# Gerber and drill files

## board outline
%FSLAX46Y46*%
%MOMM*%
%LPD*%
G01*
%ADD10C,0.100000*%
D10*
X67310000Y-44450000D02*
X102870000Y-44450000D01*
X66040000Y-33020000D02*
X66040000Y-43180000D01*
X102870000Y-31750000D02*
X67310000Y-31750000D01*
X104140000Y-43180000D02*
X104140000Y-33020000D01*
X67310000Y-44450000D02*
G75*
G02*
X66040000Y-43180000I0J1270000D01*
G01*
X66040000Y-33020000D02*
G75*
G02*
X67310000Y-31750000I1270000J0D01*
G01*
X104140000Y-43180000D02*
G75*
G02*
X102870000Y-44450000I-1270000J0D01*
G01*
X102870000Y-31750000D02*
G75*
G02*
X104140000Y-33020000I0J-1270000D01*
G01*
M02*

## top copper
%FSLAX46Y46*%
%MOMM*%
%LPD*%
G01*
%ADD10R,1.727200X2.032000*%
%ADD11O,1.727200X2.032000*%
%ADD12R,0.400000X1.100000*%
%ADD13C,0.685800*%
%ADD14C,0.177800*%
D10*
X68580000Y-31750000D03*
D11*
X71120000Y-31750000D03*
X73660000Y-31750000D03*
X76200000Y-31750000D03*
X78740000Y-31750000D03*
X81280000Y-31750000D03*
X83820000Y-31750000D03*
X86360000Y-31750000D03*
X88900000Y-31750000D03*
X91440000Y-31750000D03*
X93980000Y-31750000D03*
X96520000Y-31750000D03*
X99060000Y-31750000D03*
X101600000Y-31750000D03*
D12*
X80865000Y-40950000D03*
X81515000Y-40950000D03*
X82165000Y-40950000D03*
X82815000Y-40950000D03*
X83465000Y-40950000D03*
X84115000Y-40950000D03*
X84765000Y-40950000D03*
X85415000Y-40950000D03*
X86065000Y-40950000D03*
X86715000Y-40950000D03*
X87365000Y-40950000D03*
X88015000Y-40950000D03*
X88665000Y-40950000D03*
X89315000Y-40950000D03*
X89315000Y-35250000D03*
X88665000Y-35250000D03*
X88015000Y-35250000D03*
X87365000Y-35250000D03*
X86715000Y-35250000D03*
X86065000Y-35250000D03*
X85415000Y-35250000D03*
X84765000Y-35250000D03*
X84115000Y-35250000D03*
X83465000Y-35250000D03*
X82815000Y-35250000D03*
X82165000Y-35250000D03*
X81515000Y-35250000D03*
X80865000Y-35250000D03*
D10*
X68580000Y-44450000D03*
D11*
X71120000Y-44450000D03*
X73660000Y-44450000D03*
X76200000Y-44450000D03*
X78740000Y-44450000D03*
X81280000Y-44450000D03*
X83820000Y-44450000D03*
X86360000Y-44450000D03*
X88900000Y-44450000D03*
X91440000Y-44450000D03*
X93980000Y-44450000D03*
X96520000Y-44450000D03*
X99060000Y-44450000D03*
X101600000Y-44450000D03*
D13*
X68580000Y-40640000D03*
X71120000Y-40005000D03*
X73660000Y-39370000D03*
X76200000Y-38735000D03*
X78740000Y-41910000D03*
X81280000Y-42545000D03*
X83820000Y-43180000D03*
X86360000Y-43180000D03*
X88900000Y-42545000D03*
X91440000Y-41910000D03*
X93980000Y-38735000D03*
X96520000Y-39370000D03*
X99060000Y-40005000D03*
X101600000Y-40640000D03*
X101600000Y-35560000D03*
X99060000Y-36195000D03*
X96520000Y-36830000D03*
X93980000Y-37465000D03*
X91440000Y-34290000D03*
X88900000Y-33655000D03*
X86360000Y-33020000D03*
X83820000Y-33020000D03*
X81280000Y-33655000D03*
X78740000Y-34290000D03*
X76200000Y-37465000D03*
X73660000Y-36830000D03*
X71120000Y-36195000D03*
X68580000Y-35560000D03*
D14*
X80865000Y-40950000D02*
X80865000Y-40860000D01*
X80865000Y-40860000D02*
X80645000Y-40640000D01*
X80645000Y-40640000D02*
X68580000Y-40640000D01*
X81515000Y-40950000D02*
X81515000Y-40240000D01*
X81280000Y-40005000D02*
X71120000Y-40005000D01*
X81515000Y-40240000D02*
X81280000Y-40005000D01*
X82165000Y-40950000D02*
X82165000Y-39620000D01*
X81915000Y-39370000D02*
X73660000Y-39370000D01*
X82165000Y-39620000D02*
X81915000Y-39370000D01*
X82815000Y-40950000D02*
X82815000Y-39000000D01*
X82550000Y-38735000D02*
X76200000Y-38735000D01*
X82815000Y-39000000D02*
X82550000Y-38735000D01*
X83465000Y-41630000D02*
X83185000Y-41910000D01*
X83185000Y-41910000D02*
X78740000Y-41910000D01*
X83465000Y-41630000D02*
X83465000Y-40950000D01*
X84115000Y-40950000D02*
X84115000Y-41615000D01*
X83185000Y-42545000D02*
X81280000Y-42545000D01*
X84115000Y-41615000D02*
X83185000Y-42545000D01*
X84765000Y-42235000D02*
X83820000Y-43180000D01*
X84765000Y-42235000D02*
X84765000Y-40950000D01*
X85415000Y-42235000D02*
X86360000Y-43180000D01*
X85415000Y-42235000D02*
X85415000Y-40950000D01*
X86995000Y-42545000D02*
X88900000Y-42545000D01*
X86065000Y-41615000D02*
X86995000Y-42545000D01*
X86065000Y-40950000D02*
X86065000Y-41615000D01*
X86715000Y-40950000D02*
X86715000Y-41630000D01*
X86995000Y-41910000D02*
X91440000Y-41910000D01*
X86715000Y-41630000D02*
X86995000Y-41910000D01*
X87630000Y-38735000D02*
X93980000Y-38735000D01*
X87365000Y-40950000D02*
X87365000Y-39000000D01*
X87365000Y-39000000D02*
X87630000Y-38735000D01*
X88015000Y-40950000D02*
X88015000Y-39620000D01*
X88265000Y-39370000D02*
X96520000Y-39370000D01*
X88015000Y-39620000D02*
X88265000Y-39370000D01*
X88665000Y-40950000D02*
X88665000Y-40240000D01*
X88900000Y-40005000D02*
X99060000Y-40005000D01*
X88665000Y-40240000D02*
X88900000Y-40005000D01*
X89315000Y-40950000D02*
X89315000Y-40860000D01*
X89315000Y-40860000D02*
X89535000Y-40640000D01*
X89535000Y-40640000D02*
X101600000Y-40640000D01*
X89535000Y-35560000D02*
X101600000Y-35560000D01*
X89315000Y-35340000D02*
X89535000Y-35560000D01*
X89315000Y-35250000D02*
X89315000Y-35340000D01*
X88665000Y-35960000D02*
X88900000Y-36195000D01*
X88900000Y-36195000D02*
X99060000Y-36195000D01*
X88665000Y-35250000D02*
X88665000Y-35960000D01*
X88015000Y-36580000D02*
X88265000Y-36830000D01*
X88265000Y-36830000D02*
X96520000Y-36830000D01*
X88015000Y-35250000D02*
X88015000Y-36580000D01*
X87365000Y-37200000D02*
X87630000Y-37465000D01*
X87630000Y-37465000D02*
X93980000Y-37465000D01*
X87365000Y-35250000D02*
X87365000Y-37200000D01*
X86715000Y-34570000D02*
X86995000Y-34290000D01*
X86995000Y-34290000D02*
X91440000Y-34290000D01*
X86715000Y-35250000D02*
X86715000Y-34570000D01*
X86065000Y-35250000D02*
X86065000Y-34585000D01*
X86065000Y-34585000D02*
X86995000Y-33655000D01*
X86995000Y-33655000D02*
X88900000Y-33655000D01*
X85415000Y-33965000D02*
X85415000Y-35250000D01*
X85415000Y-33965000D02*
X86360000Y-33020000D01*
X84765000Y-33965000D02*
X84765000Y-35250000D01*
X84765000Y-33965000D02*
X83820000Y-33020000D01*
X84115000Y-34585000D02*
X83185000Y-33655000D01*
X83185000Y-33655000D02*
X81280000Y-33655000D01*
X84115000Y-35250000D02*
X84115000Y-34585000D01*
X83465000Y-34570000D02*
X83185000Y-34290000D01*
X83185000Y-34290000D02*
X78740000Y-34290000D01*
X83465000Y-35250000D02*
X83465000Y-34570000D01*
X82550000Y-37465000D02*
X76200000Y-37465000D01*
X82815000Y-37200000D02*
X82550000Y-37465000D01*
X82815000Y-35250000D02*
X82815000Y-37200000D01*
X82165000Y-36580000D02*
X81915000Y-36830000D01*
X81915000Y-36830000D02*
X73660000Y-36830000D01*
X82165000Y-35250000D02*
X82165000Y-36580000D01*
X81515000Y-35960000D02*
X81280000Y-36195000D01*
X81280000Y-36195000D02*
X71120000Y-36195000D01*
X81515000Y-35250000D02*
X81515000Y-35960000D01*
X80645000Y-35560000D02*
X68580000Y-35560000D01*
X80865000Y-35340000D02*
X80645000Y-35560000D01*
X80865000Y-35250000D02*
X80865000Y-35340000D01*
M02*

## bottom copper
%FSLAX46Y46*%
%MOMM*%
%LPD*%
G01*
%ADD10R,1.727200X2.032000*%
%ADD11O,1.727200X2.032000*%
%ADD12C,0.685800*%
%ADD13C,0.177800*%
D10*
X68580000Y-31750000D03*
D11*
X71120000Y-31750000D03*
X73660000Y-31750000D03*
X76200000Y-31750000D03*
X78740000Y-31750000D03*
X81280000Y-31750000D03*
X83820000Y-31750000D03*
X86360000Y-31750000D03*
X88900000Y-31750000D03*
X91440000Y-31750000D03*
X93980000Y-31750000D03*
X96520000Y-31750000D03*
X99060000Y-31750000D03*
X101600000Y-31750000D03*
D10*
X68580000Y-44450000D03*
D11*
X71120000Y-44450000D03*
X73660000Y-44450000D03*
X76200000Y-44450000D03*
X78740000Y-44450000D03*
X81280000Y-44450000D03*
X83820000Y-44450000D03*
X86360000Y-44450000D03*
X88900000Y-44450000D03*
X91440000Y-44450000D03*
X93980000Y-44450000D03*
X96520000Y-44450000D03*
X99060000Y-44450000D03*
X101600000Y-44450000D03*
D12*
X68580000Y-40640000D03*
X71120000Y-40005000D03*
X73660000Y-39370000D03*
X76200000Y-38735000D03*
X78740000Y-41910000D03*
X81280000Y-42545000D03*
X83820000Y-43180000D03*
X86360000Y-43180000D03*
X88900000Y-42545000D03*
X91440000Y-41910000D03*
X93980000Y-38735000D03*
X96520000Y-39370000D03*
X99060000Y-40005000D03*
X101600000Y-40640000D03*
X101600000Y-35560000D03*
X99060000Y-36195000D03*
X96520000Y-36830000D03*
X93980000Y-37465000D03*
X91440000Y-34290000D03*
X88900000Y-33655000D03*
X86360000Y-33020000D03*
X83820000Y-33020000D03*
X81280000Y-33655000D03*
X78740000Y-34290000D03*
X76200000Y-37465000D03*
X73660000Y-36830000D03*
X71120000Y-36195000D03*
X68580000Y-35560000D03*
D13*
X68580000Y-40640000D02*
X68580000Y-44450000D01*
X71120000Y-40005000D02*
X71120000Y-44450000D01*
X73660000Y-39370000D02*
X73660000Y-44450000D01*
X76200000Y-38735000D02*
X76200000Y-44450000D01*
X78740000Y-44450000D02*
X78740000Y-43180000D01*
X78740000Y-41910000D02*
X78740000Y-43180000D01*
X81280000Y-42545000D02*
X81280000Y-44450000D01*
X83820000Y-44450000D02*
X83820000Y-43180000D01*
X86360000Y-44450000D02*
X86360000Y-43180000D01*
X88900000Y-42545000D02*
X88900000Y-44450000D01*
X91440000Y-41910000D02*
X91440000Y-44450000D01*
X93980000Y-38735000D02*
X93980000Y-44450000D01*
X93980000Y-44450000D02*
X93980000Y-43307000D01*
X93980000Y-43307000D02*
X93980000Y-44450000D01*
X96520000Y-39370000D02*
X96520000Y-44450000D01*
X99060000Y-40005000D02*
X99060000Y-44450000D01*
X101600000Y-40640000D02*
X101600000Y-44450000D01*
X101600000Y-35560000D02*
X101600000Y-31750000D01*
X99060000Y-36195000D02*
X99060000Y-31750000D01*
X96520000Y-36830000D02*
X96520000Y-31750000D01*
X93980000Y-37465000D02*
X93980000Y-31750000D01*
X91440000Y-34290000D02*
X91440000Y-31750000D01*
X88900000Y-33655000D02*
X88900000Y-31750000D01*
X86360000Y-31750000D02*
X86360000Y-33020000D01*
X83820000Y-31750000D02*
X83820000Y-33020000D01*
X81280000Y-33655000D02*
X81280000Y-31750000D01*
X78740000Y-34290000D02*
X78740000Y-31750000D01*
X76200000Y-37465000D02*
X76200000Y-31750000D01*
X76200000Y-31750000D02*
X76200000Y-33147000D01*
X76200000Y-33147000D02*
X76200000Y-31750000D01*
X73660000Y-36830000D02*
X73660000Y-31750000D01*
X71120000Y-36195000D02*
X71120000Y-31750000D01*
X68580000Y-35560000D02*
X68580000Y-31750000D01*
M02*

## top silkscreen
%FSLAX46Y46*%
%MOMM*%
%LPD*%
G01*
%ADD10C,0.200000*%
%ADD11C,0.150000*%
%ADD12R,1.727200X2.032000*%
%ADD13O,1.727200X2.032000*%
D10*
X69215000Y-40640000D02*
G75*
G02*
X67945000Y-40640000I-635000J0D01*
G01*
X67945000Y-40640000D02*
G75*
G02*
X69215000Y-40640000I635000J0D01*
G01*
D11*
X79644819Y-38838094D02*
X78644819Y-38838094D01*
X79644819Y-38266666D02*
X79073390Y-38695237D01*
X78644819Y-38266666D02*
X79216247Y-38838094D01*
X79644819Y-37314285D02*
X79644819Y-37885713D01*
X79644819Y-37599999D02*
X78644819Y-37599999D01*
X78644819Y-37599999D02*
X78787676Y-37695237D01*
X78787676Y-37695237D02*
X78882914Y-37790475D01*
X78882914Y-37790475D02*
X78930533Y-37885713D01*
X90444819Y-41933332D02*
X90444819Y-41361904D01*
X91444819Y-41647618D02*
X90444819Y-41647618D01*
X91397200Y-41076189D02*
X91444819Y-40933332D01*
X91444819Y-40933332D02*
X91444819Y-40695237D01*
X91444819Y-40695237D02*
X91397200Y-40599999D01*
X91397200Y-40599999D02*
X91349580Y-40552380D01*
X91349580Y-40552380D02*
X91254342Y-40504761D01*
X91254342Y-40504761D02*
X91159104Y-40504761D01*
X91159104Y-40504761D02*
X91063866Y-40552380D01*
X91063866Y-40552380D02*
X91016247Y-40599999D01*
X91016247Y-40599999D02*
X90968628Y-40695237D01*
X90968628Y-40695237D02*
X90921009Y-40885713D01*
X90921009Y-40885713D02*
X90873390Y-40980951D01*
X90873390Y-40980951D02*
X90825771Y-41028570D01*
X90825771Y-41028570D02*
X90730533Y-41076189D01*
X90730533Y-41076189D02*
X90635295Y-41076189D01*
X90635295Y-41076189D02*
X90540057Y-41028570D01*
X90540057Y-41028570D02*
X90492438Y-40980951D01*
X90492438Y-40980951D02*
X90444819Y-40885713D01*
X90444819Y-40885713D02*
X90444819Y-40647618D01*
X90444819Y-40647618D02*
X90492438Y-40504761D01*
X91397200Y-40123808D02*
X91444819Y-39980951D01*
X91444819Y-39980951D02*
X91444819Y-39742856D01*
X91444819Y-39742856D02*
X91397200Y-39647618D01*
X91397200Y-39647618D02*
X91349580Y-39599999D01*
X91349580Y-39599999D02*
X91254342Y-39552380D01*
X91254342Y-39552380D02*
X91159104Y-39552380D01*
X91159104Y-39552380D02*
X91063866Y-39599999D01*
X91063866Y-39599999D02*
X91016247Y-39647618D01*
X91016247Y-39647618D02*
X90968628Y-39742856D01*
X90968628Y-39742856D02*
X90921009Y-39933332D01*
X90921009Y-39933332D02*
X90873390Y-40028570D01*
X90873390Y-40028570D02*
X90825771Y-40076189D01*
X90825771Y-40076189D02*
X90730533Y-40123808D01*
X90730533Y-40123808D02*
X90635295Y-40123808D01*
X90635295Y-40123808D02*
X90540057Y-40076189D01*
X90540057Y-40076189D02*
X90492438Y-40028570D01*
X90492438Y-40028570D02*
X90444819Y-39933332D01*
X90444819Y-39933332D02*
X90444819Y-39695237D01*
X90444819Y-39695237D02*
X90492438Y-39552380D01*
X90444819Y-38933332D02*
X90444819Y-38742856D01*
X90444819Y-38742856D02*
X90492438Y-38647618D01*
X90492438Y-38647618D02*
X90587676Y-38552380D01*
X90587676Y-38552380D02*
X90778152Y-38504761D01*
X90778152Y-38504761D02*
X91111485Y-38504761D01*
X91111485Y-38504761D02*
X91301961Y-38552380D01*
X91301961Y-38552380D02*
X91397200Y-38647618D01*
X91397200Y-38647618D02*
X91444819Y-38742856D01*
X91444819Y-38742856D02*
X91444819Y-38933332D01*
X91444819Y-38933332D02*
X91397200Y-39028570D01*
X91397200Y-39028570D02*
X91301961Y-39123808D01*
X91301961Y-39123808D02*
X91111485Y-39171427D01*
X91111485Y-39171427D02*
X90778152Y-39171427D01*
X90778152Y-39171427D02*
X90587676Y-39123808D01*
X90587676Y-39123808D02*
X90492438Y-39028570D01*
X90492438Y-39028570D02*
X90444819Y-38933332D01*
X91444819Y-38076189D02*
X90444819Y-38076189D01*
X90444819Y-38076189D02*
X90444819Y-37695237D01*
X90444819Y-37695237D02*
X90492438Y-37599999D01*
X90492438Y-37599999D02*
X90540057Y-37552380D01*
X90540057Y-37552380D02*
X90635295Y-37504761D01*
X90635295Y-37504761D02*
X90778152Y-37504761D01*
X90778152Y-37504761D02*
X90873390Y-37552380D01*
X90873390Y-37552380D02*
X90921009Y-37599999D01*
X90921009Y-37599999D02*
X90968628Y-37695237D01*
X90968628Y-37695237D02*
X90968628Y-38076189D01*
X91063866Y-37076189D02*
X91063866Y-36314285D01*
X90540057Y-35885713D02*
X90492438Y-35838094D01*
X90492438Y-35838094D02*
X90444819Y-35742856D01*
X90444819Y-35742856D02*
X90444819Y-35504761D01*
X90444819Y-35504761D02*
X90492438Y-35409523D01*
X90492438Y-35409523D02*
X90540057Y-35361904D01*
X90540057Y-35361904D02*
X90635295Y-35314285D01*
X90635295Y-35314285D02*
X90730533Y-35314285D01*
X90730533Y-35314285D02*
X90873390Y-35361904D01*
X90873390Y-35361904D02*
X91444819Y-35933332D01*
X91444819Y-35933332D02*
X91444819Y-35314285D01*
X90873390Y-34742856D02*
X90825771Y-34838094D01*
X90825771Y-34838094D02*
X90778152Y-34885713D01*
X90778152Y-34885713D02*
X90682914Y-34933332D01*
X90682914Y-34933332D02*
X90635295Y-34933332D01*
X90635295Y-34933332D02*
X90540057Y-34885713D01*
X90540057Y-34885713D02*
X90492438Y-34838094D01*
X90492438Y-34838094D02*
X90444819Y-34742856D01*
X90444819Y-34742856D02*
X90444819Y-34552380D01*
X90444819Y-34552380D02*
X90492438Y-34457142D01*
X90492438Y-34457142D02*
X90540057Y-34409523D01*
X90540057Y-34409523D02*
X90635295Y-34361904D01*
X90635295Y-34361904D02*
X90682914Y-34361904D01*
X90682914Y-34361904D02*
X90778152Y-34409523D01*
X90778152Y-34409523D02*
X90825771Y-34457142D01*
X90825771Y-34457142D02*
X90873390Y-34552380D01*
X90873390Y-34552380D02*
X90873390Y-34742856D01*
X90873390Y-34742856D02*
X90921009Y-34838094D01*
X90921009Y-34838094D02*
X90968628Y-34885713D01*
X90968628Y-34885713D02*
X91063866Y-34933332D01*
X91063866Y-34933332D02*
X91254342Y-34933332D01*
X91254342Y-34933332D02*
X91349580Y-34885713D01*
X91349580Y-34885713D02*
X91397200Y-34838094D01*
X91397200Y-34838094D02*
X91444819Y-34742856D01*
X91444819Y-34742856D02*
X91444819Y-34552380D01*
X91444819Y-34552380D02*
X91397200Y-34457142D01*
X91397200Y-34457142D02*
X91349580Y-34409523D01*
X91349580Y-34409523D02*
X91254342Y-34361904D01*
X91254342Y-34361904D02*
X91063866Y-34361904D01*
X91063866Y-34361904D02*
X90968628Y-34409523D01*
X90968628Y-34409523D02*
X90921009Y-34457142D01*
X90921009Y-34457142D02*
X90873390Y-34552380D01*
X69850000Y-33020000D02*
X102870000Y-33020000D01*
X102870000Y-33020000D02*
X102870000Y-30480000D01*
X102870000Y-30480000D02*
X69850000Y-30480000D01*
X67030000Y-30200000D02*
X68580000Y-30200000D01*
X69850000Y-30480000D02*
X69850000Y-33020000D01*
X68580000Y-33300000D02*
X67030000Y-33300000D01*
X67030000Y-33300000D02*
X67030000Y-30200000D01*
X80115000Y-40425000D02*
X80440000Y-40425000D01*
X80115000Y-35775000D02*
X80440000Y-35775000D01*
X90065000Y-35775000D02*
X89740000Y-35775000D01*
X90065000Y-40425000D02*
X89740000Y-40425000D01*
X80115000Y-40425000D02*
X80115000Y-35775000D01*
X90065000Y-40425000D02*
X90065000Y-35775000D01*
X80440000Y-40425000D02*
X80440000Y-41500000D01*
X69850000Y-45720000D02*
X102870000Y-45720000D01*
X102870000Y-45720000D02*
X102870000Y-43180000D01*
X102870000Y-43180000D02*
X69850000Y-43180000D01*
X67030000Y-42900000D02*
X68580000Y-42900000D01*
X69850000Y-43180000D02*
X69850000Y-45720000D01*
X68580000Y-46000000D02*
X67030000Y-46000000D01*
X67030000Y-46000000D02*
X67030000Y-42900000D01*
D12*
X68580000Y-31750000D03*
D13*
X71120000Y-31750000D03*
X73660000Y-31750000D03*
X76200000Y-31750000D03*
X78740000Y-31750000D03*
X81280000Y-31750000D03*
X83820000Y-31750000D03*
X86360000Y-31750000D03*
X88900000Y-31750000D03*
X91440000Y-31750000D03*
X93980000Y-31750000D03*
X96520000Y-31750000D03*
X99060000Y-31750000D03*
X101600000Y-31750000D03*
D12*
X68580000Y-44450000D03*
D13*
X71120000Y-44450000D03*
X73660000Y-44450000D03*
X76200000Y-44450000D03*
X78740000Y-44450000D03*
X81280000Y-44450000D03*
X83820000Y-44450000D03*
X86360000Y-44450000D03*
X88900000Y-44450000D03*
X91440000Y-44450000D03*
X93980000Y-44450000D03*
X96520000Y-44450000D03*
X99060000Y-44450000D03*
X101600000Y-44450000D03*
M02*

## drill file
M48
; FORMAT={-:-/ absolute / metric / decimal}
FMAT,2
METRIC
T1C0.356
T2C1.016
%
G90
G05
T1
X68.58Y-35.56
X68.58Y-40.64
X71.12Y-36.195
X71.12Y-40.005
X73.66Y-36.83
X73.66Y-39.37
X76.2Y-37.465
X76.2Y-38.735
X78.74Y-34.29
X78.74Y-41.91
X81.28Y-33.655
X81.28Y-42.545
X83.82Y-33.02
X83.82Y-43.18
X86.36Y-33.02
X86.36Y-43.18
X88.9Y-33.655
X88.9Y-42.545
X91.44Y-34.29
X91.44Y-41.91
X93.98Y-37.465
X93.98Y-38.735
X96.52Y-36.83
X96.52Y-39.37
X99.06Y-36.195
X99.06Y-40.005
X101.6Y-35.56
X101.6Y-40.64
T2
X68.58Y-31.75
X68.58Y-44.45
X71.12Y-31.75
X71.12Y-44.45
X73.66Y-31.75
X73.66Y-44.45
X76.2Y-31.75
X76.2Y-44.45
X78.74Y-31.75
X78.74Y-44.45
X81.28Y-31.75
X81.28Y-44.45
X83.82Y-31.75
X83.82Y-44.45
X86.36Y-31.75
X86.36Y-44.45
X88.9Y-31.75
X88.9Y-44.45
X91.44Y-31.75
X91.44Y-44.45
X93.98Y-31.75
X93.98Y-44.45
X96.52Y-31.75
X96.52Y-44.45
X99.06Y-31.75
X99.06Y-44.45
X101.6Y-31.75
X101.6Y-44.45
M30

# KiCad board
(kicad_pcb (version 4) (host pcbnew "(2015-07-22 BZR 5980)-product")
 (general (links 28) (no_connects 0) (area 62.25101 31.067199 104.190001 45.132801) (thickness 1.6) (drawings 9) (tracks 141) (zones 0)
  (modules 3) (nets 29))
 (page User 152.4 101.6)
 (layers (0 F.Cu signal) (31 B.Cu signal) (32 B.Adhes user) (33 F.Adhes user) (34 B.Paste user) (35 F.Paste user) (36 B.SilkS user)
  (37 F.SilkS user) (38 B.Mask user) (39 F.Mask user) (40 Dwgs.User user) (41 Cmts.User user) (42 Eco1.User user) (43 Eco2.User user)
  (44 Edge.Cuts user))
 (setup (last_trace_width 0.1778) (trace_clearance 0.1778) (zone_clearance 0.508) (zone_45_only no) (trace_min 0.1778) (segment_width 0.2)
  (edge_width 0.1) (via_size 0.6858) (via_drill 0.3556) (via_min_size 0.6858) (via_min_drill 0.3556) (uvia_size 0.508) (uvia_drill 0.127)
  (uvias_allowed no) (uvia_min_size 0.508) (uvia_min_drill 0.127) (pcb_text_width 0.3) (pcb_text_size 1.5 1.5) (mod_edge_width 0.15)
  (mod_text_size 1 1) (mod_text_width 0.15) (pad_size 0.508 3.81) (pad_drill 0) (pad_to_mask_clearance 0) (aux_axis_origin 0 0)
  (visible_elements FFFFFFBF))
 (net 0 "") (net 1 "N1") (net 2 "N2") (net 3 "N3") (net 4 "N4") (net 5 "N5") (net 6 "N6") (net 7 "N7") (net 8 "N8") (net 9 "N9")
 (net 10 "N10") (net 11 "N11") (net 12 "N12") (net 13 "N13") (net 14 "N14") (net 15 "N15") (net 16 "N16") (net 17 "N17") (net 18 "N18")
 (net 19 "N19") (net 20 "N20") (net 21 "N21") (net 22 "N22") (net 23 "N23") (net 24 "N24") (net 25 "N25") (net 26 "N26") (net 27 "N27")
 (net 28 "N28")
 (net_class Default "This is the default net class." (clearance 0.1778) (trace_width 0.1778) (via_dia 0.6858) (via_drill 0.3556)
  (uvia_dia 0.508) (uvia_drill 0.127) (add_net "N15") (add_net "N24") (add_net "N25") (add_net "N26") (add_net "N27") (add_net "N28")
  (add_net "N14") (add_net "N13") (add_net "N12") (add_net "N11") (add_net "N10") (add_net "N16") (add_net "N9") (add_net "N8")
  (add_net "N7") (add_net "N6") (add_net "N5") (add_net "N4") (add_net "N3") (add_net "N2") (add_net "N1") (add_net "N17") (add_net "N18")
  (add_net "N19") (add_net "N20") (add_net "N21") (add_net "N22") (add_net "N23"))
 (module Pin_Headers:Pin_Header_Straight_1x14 (layer F.Cu) (at 68.58 31.75 90)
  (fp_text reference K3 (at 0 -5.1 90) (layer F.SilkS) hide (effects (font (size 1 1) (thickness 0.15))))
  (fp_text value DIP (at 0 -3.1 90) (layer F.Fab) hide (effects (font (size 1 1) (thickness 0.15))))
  (fp_line (start -1.27 1.27) (end -1.27 34.29) (layer F.SilkS) (width 0.15))
  (fp_line (start -1.27 34.29) (end 1.27 34.29) (layer F.SilkS) (width 0.15))
  (fp_line (start 1.27 34.29) (end 1.27 1.27) (layer F.SilkS) (width 0.15))
  (fp_line (start 1.55 -1.55) (end 1.55 0) (layer F.SilkS) (width 0.15))
  (fp_line (start 1.27 1.27) (end -1.27 1.27) (layer F.SilkS) (width 0.15))
  (fp_line (start -1.55 0) (end -1.55 -1.55) (layer F.SilkS) (width 0.15))
  (fp_line (start -1.55 -1.55) (end 1.55 -1.55) (layer F.SilkS) (width 0.15))
  (pad 1 thru_hole rect (at 0 0 90) (size 2.032 1.7272) (drill 1.016) (layers *.Cu *.Mask F.SilkS) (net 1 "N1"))
  (pad 2 thru_hole oval (at 0 2.54 90) (size 2.032 1.7272) (drill 1.016) (layers *.Cu *.Mask F.SilkS) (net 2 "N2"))
  (pad 3 thru_hole oval (at 0 5.08 90) (size 2.032 1.7272) (drill 1.016) (layers *.Cu *.Mask F.SilkS) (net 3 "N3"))
  (pad 4 thru_hole oval (at 0 7.62 90) (size 2.032 1.7272) (drill 1.016) (layers *.Cu *.Mask F.SilkS) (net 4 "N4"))
  (pad 5 thru_hole oval (at 0 10.16 90) (size 2.032 1.7272) (drill 1.016) (layers *.Cu *.Mask F.SilkS) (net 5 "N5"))
  (pad 6 thru_hole oval (at 0 12.7 90) (size 2.032 1.7272) (drill 1.016) (layers *.Cu *.Mask F.SilkS) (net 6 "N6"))
  (pad 7 thru_hole oval (at 0 15.24 90) (size 2.032 1.7272) (drill 1.016) (layers *.Cu *.Mask F.SilkS) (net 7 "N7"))
  (pad 8 thru_hole oval (at 0 17.78 90) (size 2.032 1.7272) (drill 1.016) (layers *.Cu *.Mask F.SilkS) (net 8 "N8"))
  (pad 9 thru_hole oval (at 0 20.32 90) (size 2.032 1.7272) (drill 1.016) (layers *.Cu *.Mask F.SilkS) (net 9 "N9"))
  (pad 10 thru_hole oval (at 0 22.86 90) (size 2.032 1.7272) (drill 1.016) (layers *.Cu *.Mask F.SilkS) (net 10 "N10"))
  (pad 11 thru_hole oval (at 0 25.4 90) (size 2.032 1.7272) (drill 1.016) (layers *.Cu *.Mask F.SilkS) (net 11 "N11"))
  (pad 12 thru_hole oval (at 0 27.94 90) (size 2.032 1.7272) (drill 1.016) (layers *.Cu *.Mask F.SilkS) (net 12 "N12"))
  (pad 13 thru_hole oval (at 0 30.48 90) (size 2.032 1.7272) (drill 1.016) (layers *.Cu *.Mask F.SilkS) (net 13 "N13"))
  (pad 14 thru_hole oval (at 0 33.02 90) (size 2.032 1.7272) (drill 1.016) (layers *.Cu *.Mask F.SilkS) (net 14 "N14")))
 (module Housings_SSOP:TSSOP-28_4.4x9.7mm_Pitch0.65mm (layer F.Cu) (at 85.09 38.1 90)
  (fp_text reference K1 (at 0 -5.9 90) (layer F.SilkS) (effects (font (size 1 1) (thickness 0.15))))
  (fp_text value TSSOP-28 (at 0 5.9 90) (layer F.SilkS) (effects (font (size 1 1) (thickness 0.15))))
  (fp_line (start -2.325 -4.975) (end -2.325 -4.65) (layer F.SilkS) (width 0.15))
  (fp_line (start 2.325 -4.975) (end 2.325 -4.65) (layer F.SilkS) (width 0.15))
  (fp_line (start 2.325 4.975) (end 2.325 4.65) (layer F.SilkS) (width 0.15))
  (fp_line (start -2.325 4.975) (end -2.325 4.65) (layer F.SilkS) (width 0.15))
  (fp_line (start -2.325 -4.975) (end 2.325 -4.975) (layer F.SilkS) (width 0.15))
  (fp_line (start -2.325 4.975) (end 2.325 4.975) (layer F.SilkS) (width 0.15))
  (fp_line (start -2.325 -4.65) (end -3.4 -4.65) (layer F.SilkS) (width 0.15))
  (pad 1 smd rect (at -2.85 -4.225 90) (size 1.1 0.4) (layers F.Cu F.Paste F.Mask) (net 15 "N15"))
  (pad 2 smd rect (at -2.85 -3.575 90) (size 1.1 0.4) (layers F.Cu F.Paste F.Mask) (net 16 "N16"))
  (pad 3 smd rect (at -2.85 -2.925 90) (size 1.1 0.4) (layers F.Cu F.Paste F.Mask) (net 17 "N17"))
  (pad 4 smd rect (at -2.85 -2.275 90) (size 1.1 0.4) (layers F.Cu F.Paste F.Mask) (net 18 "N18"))
  (pad 5 smd rect (at -2.85 -1.625 90) (size 1.1 0.4) (layers F.Cu F.Paste F.Mask) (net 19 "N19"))
  (pad 6 smd rect (at -2.85 -0.975 90) (size 1.1 0.4) (layers F.Cu F.Paste F.Mask) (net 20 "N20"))
  (pad 7 smd rect (at -2.85 -0.325 90) (size 1.1 0.4) (layers F.Cu F.Paste F.Mask) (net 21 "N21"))
  (pad 8 smd rect (at -2.85 0.325 90) (size 1.1 0.4) (layers F.Cu F.Paste F.Mask) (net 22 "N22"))
  (pad 9 smd rect (at -2.85 0.975 90) (size 1.1 0.4) (layers F.Cu F.Paste F.Mask) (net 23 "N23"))
  (pad 10 smd rect (at -2.85 1.625 90) (size 1.1 0.4) (layers F.Cu F.Paste F.Mask) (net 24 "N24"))
  (pad 11 smd rect (at -2.85 2.275 90) (size 1.1 0.4) (layers F.Cu F.Paste F.Mask) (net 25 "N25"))
  (pad 12 smd rect (at -2.85 2.925 90) (size 1.1 0.4) (layers F.Cu F.Paste F.Mask) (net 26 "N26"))
  (pad 13 smd rect (at -2.85 3.575 90) (size 1.1 0.4) (layers F.Cu F.Paste F.Mask) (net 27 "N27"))
  (pad 14 smd rect (at -2.85 4.225 90) (size 1.1 0.4) (layers F.Cu F.Paste F.Mask) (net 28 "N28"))
  (pad 15 smd rect (at 2.85 4.225 90) (size 1.1 0.4) (layers F.Cu F.Paste F.Mask) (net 14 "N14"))
  (pad 16 smd rect (at 2.85 3.575 90) (size 1.1 0.4) (layers F.Cu F.Paste F.Mask) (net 13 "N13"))
  (pad 17 smd rect (at 2.85 2.925 90) (size 1.1 0.4) (layers F.Cu F.Paste F.Mask) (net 12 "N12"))
  (pad 18 smd rect (at 2.85 2.275 90) (size 1.1 0.4) (layers F.Cu F.Paste F.Mask) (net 11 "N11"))
  (pad 19 smd rect (at 2.85 1.625 90) (size 1.1 0.4) (layers F.Cu F.Paste F.Mask) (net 10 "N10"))
  (pad 20 smd rect (at 2.85 0.975 90) (size 1.1 0.4) (layers F.Cu F.Paste F.Mask) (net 9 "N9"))
  (pad 21 smd rect (at 2.85 0.325 90) (size 1.1 0.4) (layers F.Cu F.Paste F.Mask) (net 8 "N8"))
  (pad 22 smd rect (at 2.85 -0.325 90) (size 1.1 0.4) (layers F.Cu F.Paste F.Mask) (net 7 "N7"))
  (pad 23 smd rect (at 2.85 -0.975 90) (size 1.1 0.4) (layers F.Cu F.Paste F.Mask) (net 6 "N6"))
  (pad 24 smd rect (at 2.85 -1.625 90) (size 1.1 0.4) (layers F.Cu F.Paste F.Mask) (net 5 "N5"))
  (pad 25 smd rect (at 2.85 -2.275 90) (size 1.1 0.4) (layers F.Cu F.Paste F.Mask) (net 4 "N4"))
  (pad 26 smd rect (at 2.85 -2.925 90) (size 1.1 0.4) (layers F.Cu F.Paste F.Mask) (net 3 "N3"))
  (pad 27 smd rect (at 2.85 -3.575 90) (size 1.1 0.4) (layers F.Cu F.Paste F.Mask) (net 2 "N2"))
  (pad 28 smd rect (at 2.85 -4.225 90) (size 1.1 0.4) (layers F.Cu F.Paste F.Mask) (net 1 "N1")))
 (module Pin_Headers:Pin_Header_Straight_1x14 (layer F.Cu) (at 68.58 44.45 90)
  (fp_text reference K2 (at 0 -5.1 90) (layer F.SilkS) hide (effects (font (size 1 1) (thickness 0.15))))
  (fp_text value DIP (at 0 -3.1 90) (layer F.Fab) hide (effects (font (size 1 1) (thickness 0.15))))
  (fp_line (start -1.27 1.27) (end -1.27 34.29) (layer F.SilkS) (width 0.15))
  (fp_line (start -1.27 34.29) (end 1.27 34.29) (layer F.SilkS) (width 0.15))
  (fp_line (start 1.27 34.29) (end 1.27 1.27) (layer F.SilkS) (width 0.15))
  (fp_line (start 1.55 -1.55) (end 1.55 0) (layer F.SilkS) (width 0.15))
  (fp_line (start 1.27 1.27) (end -1.27 1.27) (layer F.SilkS) (width 0.15))
  (fp_line (start -1.55 0) (end -1.55 -1.55) (layer F.SilkS) (width 0.15))
  (fp_line (start -1.55 -1.55) (end 1.55 -1.55) (layer F.SilkS) (width 0.15))
  (pad 1 thru_hole rect (at 0 0 90) (size 2.032 1.7272) (drill 1.016) (layers *.Cu *.Mask F.SilkS) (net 15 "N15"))
  (pad 2 thru_hole oval (at 0 2.54 90) (size 2.032 1.7272) (drill 1.016) (layers *.Cu *.Mask F.SilkS) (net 16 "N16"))
  (pad 3 thru_hole oval (at 0 5.08 90) (size 2.032 1.7272) (drill 1.016) (layers *.Cu *.Mask F.SilkS) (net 17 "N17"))
  (pad 4 thru_hole oval (at 0 7.62 90) (size 2.032 1.7272) (drill 1.016) (layers *.Cu *.Mask F.SilkS) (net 18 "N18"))
  (pad 5 thru_hole oval (at 0 10.16 90) (size 2.032 1.7272) (drill 1.016) (layers *.Cu *.Mask F.SilkS) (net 19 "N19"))
  (pad 6 thru_hole oval (at 0 12.7 90) (size 2.032 1.7272) (drill 1.016) (layers *.Cu *.Mask F.SilkS) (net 20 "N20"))
  (pad 7 thru_hole oval (at 0 15.24 90) (size 2.032 1.7272) (drill 1.016) (layers *.Cu *.Mask F.SilkS) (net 21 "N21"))
  (pad 8 thru_hole oval (at 0 17.78 90) (size 2.032 1.7272) (drill 1.016) (layers *.Cu *.Mask F.SilkS) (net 22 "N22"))
  (pad 9 thru_hole oval (at 0 20.32 90) (size 2.032 1.7272) (drill 1.016) (layers *.Cu *.Mask F.SilkS) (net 23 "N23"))
  (pad 10 thru_hole oval (at 0 22.86 90) (size 2.032 1.7272) (drill 1.016) (layers *.Cu *.Mask F.SilkS) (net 24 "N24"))
  (pad 11 thru_hole oval (at 0 25.4 90) (size 2.032 1.7272) (drill 1.016) (layers *.Cu *.Mask F.SilkS) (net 25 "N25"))
  (pad 12 thru_hole oval (at 0 27.94 90) (size 2.032 1.7272) (drill 1.016) (layers *.Cu *.Mask F.SilkS) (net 26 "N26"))
  (pad 13 thru_hole oval (at 0 30.48 90) (size 2.032 1.7272) (drill 1.016) (layers *.Cu *.Mask F.SilkS) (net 27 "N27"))
  (pad 14 thru_hole oval (at 0 33.02 90) (size 2.032 1.7272) (drill 1.016) (layers *.Cu *.Mask F.SilkS) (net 28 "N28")))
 (gr_circle (center 68.58 40.64) (end 68.58 40.005) (layer F.SilkS) (width 0.2))
 (gr_line (start 67.31 44.45) (end 102.87 44.45) (angle 90) (layer Edge.Cuts) (width 0.1))
 (gr_line (start 66.04 33.02) (end 66.04 43.18) (angle 90) (layer Edge.Cuts) (width 0.1))
 (gr_line (start 102.87 31.75) (end 67.31 31.75) (angle 90) (layer Edge.Cuts) (width 0.1))
 (gr_line (start 104.14 43.18) (end 104.14 33.02) (angle 90) (layer Edge.Cuts) (width 0.1))
 (gr_arc (start 67.31 43.18) (end 67.31 44.45) (angle 90) (layer Edge.Cuts) (width 0.1))
 (gr_arc (start 67.31 33.02) (end 66.04 33.02) (angle 90) (layer Edge.Cuts) (width 0.1))
 (gr_arc (start 102.87 43.18) (end 104.14 43.18) (angle 90) (layer Edge.Cuts) (width 0.1))
 (gr_arc (start 102.87 33.02) (end 102.87 31.75) (angle 90) (layer Edge.Cuts) (width 0.1))
 (segment (start 80.865 40.95) (end 80.865 40.86) (width 0.1778) (layer F.Cu) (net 15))
 (segment (start 80.865 40.86) (end 80.645 40.64) (width 0.1778) (layer F.Cu) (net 15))
 (segment (start 68.58 40.64) (end 68.58 44.45) (width 0.1778) (layer B.Cu) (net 15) (status 800000))
 (via (at 68.58 40.64) (size 0.6858) (drill 0.3556) (layers F.Cu B.Cu) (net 15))
 (segment (start 80.645 40.64) (end 68.58 40.64) (width 0.1778) (layer F.Cu) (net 15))
 (segment (start 81.515 40.95) (end 81.515 40.24) (width 0.1778) (layer F.Cu) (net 16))
 (segment (start 71.12 40.005) (end 71.12 44.45) (width 0.1778) (layer B.Cu) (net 16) (status 800000))
 (via (at 71.12 40.005) (size 0.6858) (drill 0.3556) (layers F.Cu B.Cu) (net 16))
 (segment (start 81.28 40.005) (end 71.12 40.005) (width 0.1778) (layer F.Cu) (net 16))
 (segment (start 81.515 40.24) (end 81.28 40.005) (width 0.1778) (layer F.Cu) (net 16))
 (segment (start 82.165 40.95) (end 82.165 39.62) (width 0.1778) (layer F.Cu) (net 17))
 (segment (start 73.66 39.37) (end 73.66 44.45) (width 0.1778) (layer B.Cu) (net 17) (status 800000))
 (via (at 73.66 39.37) (size 0.6858) (drill 0.3556) (layers F.Cu B.Cu) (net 17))
 (segment (start 81.915 39.37) (end 73.66 39.37) (width 0.1778) (layer F.Cu) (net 17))
 (segment (start 82.165 39.62) (end 81.915 39.37) (width 0.1778) (layer F.Cu) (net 17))
 (segment (start 82.815 40.95) (end 82.815 39) (width 0.1778) (layer F.Cu) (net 18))
 (segment (start 76.2 38.735) (end 76.2 44.45) (width 0.1778) (layer B.Cu) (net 18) (status 800000))
 (via (at 76.2 38.735) (size 0.6858) (drill 0.3556) (layers F.Cu B.Cu) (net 18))
 (segment (start 82.55 38.735) (end 76.2 38.735) (width 0.1778) (layer F.Cu) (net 18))
 (segment (start 82.815 39) (end 82.55 38.735) (width 0.1778) (layer F.Cu) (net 18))
 (segment (start 78.74 44.45) (end 78.74 43.18) (width 0.1778) (layer B.Cu) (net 19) (status 400000))
 (segment (start 83.465 41.63) (end 83.185 41.91) (width 0.1778) (layer F.Cu) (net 19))
 (segment (start 83.185 41.91) (end 78.74 41.91) (width 0.1778) (layer F.Cu) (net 19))
 (via (at 78.74 41.91) (size 0.6858) (drill 0.3556) (layers F.Cu B.Cu) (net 19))
 (segment (start 78.74 41.91) (end 78.74 43.18) (width 0.1778) (layer B.Cu) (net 19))
 (segment (start 83.465 41.63) (end 83.465 40.95) (width 0.1778) (layer F.Cu) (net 19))
 (segment (start 84.115 40.95) (end 84.115 41.615) (width 0.1778) (layer F.Cu) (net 20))
 (segment (start 81.28 42.545) (end 81.28 44.45) (width 0.1778) (layer B.Cu) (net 20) (status 800000))
 (via (at 81.28 42.545) (size 0.6858) (drill 0.3556) (layers F.Cu B.Cu) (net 20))
 (segment (start 83.185 42.545) (end 81.28 42.545) (width 0.1778) (layer F.Cu) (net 20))
 (segment (start 84.115 41.615) (end 83.185 42.545) (width 0.1778) (layer F.Cu) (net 20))
 (segment (start 83.82 44.45) (end 83.82 43.18) (width 0.1778) (layer B.Cu) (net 21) (status 400000))
 (segment (start 84.765 42.235) (end 83.82 43.18) (width 0.1778) (layer F.Cu) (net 21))
 (via (at 83.82 43.18) (size 0.6858) (drill 0.3556) (layers F.Cu B.Cu) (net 21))
 (segment (start 84.765 42.235) (end 84.765 40.95) (width 0.1778) (layer F.Cu) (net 21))
 (segment (start 86.36 44.45) (end 86.36 43.18) (width 0.1778) (layer B.Cu) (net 22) (status 400000))
 (segment (start 85.415 42.235) (end 86.36 43.18) (width 0.1778) (layer F.Cu) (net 22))
 (via (at 86.36 43.18) (size 0.6858) (drill 0.3556) (layers F.Cu B.Cu) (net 22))
 (segment (start 85.415 42.235) (end 85.415 40.95) (width 0.1778) (layer F.Cu) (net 22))
 (segment (start 86.995 42.545) (end 88.9 42.545) (width 0.1778) (layer F.Cu) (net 23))
 (segment (start 86.065 41.615) (end 86.995 42.545) (width 0.1778) (layer F.Cu) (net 23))
 (segment (start 86.065 40.95) (end 86.065 41.615) (width 0.1778) (layer F.Cu) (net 23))
 (segment (start 88.9 42.545) (end 88.9 44.45) (width 0.1778) (layer B.Cu) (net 23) (status 800000))
 (via (at 88.9 42.545) (size 0.6858) (drill 0.3556) (layers F.Cu B.Cu) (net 23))
 (segment (start 86.715 40.95) (end 86.715 41.63) (width 0.1778) (layer F.Cu) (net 24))
 (segment (start 91.44 41.91) (end 91.44 44.45) (width 0.1778) (layer B.Cu) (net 24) (status 800000))
 (via (at 91.44 41.91) (size 0.6858) (drill 0.3556) (layers F.Cu B.Cu) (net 24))
 (segment (start 86.995 41.91) (end 91.44 41.91) (width 0.1778) (layer F.Cu) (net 24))
 (segment (start 86.715 41.63) (end 86.995 41.91) (width 0.1778) (layer F.Cu) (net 24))
 (segment (start 87.63 38.735) (end 93.98 38.735) (width 0.1778) (layer F.Cu) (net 25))
 (segment (start 93.98 38.735) (end 93.98 44.45) (width 0.1778) (layer B.Cu) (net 25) (status 800000))
 (via (at 93.98 38.735) (size 0.6858) (drill 0.3556) (layers F.Cu B.Cu) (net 25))
 (segment (start 93.98 44.45) (end 93.98 43.307) (width 0.1778) (layer B.Cu) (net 25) (status 400000))
 (segment (start 93.98 43.307) (end 93.98 44.45) (width 0.1778) (layer B.Cu) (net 25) (status 800000))
 (segment (start 87.365 40.95) (end 87.365 39) (width 0.1778) (layer F.Cu) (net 25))
 (segment (start 87.365 39) (end 87.63 38.735) (width 0.1778) (layer F.Cu) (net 25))
 (segment (start 88.015 40.95) (end 88.015 39.62) (width 0.1778) (layer F.Cu) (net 26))
 (segment (start 96.52 39.37) (end 96.52 44.45) (width 0.1778) (layer B.Cu) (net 26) (status 800000))
 (via (at 96.52 39.37) (size 0.6858) (drill 0.3556) (layers F.Cu B.Cu) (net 26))
 (segment (start 88.265 39.37) (end 96.52 39.37) (width 0.1778) (layer F.Cu) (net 26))
 (segment (start 88.015 39.62) (end 88.265 39.37) (width 0.1778) (layer F.Cu) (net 26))
 (segment (start 88.665 40.95) (end 88.665 40.24) (width 0.1778) (layer F.Cu) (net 27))
 (segment (start 99.06 40.005) (end 99.06 44.45) (width 0.1778) (layer B.Cu) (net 27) (status 800000))
 (via (at 99.06 40.005) (size 0.6858) (drill 0.3556) (layers F.Cu B.Cu) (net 27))
 (segment (start 88.9 40.005) (end 99.06 40.005) (width 0.1778) (layer F.Cu) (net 27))
 (segment (start 88.665 40.24) (end 88.9 40.005) (width 0.1778) (layer F.Cu) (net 27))
 (segment (start 89.315 40.95) (end 89.315 40.86) (width 0.1778) (layer F.Cu) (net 28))
 (segment (start 89.315 40.86) (end 89.535 40.64) (width 0.1778) (layer F.Cu) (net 28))
 (segment (start 89.535 40.64) (end 101.6 40.64) (width 0.1778) (layer F.Cu) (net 28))
 (via (at 101.6 40.64) (size 0.6858) (drill 0.3556) (layers F.Cu B.Cu) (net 28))
 (segment (start 101.6 40.64) (end 101.6 44.45) (width 0.1778) (layer B.Cu) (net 28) (status 800000))
 (segment (start 89.535 35.56) (end 101.6 35.56) (width 0.1778) (layer F.Cu) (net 14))
 (via (at 101.6 35.56) (size 0.6858) (drill 0.3556) (layers F.Cu B.Cu) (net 14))
 (segment (start 101.6 35.56) (end 101.6 31.75) (width 0.1778) (layer B.Cu) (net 14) (status 800000))
 (segment (start 89.315 35.34) (end 89.535 35.56) (width 0.1778) (layer F.Cu) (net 14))
 (segment (start 89.315 35.25) (end 89.315 35.34) (width 0.1778) (layer F.Cu) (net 14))
 (segment (start 88.665 35.96) (end 88.9 36.195) (width 0.1778) (layer F.Cu) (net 13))
 (segment (start 88.9 36.195) (end 99.06 36.195) (width 0.1778) (layer F.Cu) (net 13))
 (via (at 99.06 36.195) (size 0.6858) (drill 0.3556) (layers F.Cu B.Cu) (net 13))
 (segment (start 99.06 36.195) (end 99.06 31.75) (width 0.1778) (layer B.Cu) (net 13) (status 800000))
 (segment (start 88.665 35.25) (end 88.665 35.96) (width 0.1778) (layer F.Cu) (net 13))
 (segment (start 88.015 36.58) (end 88.265 36.83) (width 0.1778) (layer F.Cu) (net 12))
 (segment (start 88.265 36.83) (end 96.52 36.83) (width 0.1778) (layer F.Cu) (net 12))
 (via (at 96.52 36.83) (size 0.6858) (drill 0.3556) (layers F.Cu B.Cu) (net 12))
 (segment (start 96.52 36.83) (end 96.52 31.75) (width 0.1778) (layer B.Cu) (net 12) (status 800000))
 (segment (start 88.015 35.25) (end 88.015 36.58) (width 0.1778) (layer F.Cu) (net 12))
 (segment (start 87.365 37.2) (end 87.63 37.465) (width 0.1778) (layer F.Cu) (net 11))
 (segment (start 87.63 37.465) (end 93.98 37.465) (width 0.1778) (layer F.Cu) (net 11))
 (via (at 93.98 37.465) (size 0.6858) (drill 0.3556) (layers F.Cu B.Cu) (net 11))
 (segment (start 93.98 37.465) (end 93.98 31.75) (width 0.1778) (layer B.Cu) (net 11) (status 800000))
 (segment (start 87.365 35.25) (end 87.365 37.2) (width 0.1778) (layer F.Cu) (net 11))
 (segment (start 86.715 34.57) (end 86.995 34.29) (width 0.1778) (layer F.Cu) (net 10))
 (segment (start 86.995 34.29) (end 91.44 34.29) (width 0.1778) (layer F.Cu) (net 10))
 (via (at 91.44 34.29) (size 0.6858) (drill 0.3556) (layers F.Cu B.Cu) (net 10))
 (segment (start 91.44 34.29) (end 91.44 31.75) (width 0.1778) (layer B.Cu) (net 10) (status 800000))
 (segment (start 86.715 35.25) (end 86.715 34.57) (width 0.1778) (layer F.Cu) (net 10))
 (via (at 88.9 33.655) (size 0.6858) (drill 0.3556) (layers F.Cu B.Cu) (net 9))
 (segment (start 88.9 33.655) (end 88.9 31.75) (width 0.1778) (layer B.Cu) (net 9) (status 800000))
 (segment (start 86.065 35.25) (end 86.065 34.585) (width 0.1778) (layer F.Cu) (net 9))
 (segment (start 86.065 34.585) (end 86.995 33.655) (width 0.1778) (layer F.Cu) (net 9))
 (segment (start 86.995 33.655) (end 88.9 33.655) (width 0.1778) (layer F.Cu) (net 9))
 (segment (start 86.36 31.75) (end 86.36 33.02) (width 0.1778) (layer B.Cu) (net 8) (status 400000))
 (segment (start 85.415 33.965) (end 85.415 35.25) (width 0.1778) (layer F.Cu) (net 8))
 (via (at 86.36 33.02) (size 0.6858) (drill 0.3556) (layers F.Cu B.Cu) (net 8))
 (segment (start 85.415 33.965) (end 86.36 33.02) (width 0.1778) (layer F.Cu) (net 8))
 (segment (start 83.82 31.75) (end 83.82 33.02) (width 0.1778) (layer B.Cu) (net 7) (status 400000))
 (segment (start 84.765 33.965) (end 84.765 35.25) (width 0.1778) (layer F.Cu) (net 7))
 (via (at 83.82 33.02) (size 0.6858) (drill 0.3556) (layers F.Cu B.Cu) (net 7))
 (segment (start 84.765 33.965) (end 83.82 33.02) (width 0.1778) (layer F.Cu) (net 7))
 (segment (start 84.115 34.585) (end 83.185 33.655) (width 0.1778) (layer F.Cu) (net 6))
 (segment (start 83.185 33.655) (end 81.28 33.655) (width 0.1778) (layer F.Cu) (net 6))
 (via (at 81.28 33.655) (size 0.6858) (drill 0.3556) (layers F.Cu B.Cu) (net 6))
 (segment (start 81.28 33.655) (end 81.28 31.75) (width 0.1778) (layer B.Cu) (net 6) (status 800000))
 (segment (start 84.115 35.25) (end 84.115 34.585) (width 0.1778) (layer F.Cu) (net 6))
 (segment (start 83.465 34.57) (end 83.185 34.29) (width 0.1778) (layer F.Cu) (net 5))
 (segment (start 83.185 34.29) (end 78.74 34.29) (width 0.1778) (layer F.Cu) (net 5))
 (via (at 78.74 34.29) (size 0.6858) (drill 0.3556) (layers F.Cu B.Cu) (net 5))
 (segment (start 78.74 34.29) (end 78.74 31.75) (width 0.1778) (layer B.Cu) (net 5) (status 800000))
 (segment (start 83.465 35.25) (end 83.465 34.57) (width 0.1778) (layer F.Cu) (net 5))
 (segment (start 82.55 37.465) (end 76.2 37.465) (width 0.1778) (layer F.Cu) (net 4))
 (segment (start 76.2 37.465) (end 76.2 31.75) (width 0.1778) (layer B.Cu) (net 4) (status 800000))
 (via (at 76.2 37.465) (size 0.6858) (drill 0.3556) (layers F.Cu B.Cu) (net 4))
 (segment (start 76.2 31.75) (end 76.2 33.147) (width 0.1778) (layer B.Cu) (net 4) (status 400000))
 (segment (start 76.2 33.147) (end 76.2 31.75) (width 0.1778) (layer B.Cu) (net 4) (status 800000))
 (segment (start 82.815 37.2) (end 82.55 37.465) (width 0.1778) (layer F.Cu) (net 4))
 (segment (start 82.815 35.25) (end 82.815 37.2) (width 0.1778) (layer F.Cu) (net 4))
 (segment (start 82.165 36.58) (end 81.915 36.83) (width 0.1778) (layer F.Cu) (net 3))
 (segment (start 81.915 36.83) (end 73.66 36.83) (width 0.1778) (layer F.Cu) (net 3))
 (via (at 73.66 36.83) (size 0.6858) (drill 0.3556) (layers F.Cu B.Cu) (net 3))
 (segment (start 73.66 36.83) (end 73.66 31.75) (width 0.1778) (layer B.Cu) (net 3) (status 800000))
 (segment (start 82.165 35.25) (end 82.165 36.58) (width 0.1778) (layer F.Cu) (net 3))
 (segment (start 81.515 35.96) (end 81.28 36.195) (width 0.1778) (layer F.Cu) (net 2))
 (segment (start 81.28 36.195) (end 71.12 36.195) (width 0.1778) (layer F.Cu) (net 2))
 (via (at 71.12 36.195) (size 0.6858) (drill 0.3556) (layers F.Cu B.Cu) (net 2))
 (segment (start 71.12 36.195) (end 71.12 31.75) (width 0.1778) (layer B.Cu) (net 2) (status 800000))
 (segment (start 81.515 35.25) (end 81.515 35.96) (width 0.1778) (layer F.Cu) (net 2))
 (segment (start 68.58 35.56) (end 68.58 31.75) (width 0.1778) (layer B.Cu) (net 1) (status 800000))
 (via (at 68.58 35.56) (size 0.6858) (drill 0.3556) (layers F.Cu B.Cu) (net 1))
 (segment (start 80.645 35.56) (end 68.58 35.56) (width 0.1778) (layer F.Cu) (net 1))
 (segment (start 80.865 35.34) (end 80.645 35.56) (width 0.1778) (layer F.Cu) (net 1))
 (segment (start 80.865 35.25) (end 80.865 35.34) (width 0.1778) (layer F.Cu) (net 1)))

